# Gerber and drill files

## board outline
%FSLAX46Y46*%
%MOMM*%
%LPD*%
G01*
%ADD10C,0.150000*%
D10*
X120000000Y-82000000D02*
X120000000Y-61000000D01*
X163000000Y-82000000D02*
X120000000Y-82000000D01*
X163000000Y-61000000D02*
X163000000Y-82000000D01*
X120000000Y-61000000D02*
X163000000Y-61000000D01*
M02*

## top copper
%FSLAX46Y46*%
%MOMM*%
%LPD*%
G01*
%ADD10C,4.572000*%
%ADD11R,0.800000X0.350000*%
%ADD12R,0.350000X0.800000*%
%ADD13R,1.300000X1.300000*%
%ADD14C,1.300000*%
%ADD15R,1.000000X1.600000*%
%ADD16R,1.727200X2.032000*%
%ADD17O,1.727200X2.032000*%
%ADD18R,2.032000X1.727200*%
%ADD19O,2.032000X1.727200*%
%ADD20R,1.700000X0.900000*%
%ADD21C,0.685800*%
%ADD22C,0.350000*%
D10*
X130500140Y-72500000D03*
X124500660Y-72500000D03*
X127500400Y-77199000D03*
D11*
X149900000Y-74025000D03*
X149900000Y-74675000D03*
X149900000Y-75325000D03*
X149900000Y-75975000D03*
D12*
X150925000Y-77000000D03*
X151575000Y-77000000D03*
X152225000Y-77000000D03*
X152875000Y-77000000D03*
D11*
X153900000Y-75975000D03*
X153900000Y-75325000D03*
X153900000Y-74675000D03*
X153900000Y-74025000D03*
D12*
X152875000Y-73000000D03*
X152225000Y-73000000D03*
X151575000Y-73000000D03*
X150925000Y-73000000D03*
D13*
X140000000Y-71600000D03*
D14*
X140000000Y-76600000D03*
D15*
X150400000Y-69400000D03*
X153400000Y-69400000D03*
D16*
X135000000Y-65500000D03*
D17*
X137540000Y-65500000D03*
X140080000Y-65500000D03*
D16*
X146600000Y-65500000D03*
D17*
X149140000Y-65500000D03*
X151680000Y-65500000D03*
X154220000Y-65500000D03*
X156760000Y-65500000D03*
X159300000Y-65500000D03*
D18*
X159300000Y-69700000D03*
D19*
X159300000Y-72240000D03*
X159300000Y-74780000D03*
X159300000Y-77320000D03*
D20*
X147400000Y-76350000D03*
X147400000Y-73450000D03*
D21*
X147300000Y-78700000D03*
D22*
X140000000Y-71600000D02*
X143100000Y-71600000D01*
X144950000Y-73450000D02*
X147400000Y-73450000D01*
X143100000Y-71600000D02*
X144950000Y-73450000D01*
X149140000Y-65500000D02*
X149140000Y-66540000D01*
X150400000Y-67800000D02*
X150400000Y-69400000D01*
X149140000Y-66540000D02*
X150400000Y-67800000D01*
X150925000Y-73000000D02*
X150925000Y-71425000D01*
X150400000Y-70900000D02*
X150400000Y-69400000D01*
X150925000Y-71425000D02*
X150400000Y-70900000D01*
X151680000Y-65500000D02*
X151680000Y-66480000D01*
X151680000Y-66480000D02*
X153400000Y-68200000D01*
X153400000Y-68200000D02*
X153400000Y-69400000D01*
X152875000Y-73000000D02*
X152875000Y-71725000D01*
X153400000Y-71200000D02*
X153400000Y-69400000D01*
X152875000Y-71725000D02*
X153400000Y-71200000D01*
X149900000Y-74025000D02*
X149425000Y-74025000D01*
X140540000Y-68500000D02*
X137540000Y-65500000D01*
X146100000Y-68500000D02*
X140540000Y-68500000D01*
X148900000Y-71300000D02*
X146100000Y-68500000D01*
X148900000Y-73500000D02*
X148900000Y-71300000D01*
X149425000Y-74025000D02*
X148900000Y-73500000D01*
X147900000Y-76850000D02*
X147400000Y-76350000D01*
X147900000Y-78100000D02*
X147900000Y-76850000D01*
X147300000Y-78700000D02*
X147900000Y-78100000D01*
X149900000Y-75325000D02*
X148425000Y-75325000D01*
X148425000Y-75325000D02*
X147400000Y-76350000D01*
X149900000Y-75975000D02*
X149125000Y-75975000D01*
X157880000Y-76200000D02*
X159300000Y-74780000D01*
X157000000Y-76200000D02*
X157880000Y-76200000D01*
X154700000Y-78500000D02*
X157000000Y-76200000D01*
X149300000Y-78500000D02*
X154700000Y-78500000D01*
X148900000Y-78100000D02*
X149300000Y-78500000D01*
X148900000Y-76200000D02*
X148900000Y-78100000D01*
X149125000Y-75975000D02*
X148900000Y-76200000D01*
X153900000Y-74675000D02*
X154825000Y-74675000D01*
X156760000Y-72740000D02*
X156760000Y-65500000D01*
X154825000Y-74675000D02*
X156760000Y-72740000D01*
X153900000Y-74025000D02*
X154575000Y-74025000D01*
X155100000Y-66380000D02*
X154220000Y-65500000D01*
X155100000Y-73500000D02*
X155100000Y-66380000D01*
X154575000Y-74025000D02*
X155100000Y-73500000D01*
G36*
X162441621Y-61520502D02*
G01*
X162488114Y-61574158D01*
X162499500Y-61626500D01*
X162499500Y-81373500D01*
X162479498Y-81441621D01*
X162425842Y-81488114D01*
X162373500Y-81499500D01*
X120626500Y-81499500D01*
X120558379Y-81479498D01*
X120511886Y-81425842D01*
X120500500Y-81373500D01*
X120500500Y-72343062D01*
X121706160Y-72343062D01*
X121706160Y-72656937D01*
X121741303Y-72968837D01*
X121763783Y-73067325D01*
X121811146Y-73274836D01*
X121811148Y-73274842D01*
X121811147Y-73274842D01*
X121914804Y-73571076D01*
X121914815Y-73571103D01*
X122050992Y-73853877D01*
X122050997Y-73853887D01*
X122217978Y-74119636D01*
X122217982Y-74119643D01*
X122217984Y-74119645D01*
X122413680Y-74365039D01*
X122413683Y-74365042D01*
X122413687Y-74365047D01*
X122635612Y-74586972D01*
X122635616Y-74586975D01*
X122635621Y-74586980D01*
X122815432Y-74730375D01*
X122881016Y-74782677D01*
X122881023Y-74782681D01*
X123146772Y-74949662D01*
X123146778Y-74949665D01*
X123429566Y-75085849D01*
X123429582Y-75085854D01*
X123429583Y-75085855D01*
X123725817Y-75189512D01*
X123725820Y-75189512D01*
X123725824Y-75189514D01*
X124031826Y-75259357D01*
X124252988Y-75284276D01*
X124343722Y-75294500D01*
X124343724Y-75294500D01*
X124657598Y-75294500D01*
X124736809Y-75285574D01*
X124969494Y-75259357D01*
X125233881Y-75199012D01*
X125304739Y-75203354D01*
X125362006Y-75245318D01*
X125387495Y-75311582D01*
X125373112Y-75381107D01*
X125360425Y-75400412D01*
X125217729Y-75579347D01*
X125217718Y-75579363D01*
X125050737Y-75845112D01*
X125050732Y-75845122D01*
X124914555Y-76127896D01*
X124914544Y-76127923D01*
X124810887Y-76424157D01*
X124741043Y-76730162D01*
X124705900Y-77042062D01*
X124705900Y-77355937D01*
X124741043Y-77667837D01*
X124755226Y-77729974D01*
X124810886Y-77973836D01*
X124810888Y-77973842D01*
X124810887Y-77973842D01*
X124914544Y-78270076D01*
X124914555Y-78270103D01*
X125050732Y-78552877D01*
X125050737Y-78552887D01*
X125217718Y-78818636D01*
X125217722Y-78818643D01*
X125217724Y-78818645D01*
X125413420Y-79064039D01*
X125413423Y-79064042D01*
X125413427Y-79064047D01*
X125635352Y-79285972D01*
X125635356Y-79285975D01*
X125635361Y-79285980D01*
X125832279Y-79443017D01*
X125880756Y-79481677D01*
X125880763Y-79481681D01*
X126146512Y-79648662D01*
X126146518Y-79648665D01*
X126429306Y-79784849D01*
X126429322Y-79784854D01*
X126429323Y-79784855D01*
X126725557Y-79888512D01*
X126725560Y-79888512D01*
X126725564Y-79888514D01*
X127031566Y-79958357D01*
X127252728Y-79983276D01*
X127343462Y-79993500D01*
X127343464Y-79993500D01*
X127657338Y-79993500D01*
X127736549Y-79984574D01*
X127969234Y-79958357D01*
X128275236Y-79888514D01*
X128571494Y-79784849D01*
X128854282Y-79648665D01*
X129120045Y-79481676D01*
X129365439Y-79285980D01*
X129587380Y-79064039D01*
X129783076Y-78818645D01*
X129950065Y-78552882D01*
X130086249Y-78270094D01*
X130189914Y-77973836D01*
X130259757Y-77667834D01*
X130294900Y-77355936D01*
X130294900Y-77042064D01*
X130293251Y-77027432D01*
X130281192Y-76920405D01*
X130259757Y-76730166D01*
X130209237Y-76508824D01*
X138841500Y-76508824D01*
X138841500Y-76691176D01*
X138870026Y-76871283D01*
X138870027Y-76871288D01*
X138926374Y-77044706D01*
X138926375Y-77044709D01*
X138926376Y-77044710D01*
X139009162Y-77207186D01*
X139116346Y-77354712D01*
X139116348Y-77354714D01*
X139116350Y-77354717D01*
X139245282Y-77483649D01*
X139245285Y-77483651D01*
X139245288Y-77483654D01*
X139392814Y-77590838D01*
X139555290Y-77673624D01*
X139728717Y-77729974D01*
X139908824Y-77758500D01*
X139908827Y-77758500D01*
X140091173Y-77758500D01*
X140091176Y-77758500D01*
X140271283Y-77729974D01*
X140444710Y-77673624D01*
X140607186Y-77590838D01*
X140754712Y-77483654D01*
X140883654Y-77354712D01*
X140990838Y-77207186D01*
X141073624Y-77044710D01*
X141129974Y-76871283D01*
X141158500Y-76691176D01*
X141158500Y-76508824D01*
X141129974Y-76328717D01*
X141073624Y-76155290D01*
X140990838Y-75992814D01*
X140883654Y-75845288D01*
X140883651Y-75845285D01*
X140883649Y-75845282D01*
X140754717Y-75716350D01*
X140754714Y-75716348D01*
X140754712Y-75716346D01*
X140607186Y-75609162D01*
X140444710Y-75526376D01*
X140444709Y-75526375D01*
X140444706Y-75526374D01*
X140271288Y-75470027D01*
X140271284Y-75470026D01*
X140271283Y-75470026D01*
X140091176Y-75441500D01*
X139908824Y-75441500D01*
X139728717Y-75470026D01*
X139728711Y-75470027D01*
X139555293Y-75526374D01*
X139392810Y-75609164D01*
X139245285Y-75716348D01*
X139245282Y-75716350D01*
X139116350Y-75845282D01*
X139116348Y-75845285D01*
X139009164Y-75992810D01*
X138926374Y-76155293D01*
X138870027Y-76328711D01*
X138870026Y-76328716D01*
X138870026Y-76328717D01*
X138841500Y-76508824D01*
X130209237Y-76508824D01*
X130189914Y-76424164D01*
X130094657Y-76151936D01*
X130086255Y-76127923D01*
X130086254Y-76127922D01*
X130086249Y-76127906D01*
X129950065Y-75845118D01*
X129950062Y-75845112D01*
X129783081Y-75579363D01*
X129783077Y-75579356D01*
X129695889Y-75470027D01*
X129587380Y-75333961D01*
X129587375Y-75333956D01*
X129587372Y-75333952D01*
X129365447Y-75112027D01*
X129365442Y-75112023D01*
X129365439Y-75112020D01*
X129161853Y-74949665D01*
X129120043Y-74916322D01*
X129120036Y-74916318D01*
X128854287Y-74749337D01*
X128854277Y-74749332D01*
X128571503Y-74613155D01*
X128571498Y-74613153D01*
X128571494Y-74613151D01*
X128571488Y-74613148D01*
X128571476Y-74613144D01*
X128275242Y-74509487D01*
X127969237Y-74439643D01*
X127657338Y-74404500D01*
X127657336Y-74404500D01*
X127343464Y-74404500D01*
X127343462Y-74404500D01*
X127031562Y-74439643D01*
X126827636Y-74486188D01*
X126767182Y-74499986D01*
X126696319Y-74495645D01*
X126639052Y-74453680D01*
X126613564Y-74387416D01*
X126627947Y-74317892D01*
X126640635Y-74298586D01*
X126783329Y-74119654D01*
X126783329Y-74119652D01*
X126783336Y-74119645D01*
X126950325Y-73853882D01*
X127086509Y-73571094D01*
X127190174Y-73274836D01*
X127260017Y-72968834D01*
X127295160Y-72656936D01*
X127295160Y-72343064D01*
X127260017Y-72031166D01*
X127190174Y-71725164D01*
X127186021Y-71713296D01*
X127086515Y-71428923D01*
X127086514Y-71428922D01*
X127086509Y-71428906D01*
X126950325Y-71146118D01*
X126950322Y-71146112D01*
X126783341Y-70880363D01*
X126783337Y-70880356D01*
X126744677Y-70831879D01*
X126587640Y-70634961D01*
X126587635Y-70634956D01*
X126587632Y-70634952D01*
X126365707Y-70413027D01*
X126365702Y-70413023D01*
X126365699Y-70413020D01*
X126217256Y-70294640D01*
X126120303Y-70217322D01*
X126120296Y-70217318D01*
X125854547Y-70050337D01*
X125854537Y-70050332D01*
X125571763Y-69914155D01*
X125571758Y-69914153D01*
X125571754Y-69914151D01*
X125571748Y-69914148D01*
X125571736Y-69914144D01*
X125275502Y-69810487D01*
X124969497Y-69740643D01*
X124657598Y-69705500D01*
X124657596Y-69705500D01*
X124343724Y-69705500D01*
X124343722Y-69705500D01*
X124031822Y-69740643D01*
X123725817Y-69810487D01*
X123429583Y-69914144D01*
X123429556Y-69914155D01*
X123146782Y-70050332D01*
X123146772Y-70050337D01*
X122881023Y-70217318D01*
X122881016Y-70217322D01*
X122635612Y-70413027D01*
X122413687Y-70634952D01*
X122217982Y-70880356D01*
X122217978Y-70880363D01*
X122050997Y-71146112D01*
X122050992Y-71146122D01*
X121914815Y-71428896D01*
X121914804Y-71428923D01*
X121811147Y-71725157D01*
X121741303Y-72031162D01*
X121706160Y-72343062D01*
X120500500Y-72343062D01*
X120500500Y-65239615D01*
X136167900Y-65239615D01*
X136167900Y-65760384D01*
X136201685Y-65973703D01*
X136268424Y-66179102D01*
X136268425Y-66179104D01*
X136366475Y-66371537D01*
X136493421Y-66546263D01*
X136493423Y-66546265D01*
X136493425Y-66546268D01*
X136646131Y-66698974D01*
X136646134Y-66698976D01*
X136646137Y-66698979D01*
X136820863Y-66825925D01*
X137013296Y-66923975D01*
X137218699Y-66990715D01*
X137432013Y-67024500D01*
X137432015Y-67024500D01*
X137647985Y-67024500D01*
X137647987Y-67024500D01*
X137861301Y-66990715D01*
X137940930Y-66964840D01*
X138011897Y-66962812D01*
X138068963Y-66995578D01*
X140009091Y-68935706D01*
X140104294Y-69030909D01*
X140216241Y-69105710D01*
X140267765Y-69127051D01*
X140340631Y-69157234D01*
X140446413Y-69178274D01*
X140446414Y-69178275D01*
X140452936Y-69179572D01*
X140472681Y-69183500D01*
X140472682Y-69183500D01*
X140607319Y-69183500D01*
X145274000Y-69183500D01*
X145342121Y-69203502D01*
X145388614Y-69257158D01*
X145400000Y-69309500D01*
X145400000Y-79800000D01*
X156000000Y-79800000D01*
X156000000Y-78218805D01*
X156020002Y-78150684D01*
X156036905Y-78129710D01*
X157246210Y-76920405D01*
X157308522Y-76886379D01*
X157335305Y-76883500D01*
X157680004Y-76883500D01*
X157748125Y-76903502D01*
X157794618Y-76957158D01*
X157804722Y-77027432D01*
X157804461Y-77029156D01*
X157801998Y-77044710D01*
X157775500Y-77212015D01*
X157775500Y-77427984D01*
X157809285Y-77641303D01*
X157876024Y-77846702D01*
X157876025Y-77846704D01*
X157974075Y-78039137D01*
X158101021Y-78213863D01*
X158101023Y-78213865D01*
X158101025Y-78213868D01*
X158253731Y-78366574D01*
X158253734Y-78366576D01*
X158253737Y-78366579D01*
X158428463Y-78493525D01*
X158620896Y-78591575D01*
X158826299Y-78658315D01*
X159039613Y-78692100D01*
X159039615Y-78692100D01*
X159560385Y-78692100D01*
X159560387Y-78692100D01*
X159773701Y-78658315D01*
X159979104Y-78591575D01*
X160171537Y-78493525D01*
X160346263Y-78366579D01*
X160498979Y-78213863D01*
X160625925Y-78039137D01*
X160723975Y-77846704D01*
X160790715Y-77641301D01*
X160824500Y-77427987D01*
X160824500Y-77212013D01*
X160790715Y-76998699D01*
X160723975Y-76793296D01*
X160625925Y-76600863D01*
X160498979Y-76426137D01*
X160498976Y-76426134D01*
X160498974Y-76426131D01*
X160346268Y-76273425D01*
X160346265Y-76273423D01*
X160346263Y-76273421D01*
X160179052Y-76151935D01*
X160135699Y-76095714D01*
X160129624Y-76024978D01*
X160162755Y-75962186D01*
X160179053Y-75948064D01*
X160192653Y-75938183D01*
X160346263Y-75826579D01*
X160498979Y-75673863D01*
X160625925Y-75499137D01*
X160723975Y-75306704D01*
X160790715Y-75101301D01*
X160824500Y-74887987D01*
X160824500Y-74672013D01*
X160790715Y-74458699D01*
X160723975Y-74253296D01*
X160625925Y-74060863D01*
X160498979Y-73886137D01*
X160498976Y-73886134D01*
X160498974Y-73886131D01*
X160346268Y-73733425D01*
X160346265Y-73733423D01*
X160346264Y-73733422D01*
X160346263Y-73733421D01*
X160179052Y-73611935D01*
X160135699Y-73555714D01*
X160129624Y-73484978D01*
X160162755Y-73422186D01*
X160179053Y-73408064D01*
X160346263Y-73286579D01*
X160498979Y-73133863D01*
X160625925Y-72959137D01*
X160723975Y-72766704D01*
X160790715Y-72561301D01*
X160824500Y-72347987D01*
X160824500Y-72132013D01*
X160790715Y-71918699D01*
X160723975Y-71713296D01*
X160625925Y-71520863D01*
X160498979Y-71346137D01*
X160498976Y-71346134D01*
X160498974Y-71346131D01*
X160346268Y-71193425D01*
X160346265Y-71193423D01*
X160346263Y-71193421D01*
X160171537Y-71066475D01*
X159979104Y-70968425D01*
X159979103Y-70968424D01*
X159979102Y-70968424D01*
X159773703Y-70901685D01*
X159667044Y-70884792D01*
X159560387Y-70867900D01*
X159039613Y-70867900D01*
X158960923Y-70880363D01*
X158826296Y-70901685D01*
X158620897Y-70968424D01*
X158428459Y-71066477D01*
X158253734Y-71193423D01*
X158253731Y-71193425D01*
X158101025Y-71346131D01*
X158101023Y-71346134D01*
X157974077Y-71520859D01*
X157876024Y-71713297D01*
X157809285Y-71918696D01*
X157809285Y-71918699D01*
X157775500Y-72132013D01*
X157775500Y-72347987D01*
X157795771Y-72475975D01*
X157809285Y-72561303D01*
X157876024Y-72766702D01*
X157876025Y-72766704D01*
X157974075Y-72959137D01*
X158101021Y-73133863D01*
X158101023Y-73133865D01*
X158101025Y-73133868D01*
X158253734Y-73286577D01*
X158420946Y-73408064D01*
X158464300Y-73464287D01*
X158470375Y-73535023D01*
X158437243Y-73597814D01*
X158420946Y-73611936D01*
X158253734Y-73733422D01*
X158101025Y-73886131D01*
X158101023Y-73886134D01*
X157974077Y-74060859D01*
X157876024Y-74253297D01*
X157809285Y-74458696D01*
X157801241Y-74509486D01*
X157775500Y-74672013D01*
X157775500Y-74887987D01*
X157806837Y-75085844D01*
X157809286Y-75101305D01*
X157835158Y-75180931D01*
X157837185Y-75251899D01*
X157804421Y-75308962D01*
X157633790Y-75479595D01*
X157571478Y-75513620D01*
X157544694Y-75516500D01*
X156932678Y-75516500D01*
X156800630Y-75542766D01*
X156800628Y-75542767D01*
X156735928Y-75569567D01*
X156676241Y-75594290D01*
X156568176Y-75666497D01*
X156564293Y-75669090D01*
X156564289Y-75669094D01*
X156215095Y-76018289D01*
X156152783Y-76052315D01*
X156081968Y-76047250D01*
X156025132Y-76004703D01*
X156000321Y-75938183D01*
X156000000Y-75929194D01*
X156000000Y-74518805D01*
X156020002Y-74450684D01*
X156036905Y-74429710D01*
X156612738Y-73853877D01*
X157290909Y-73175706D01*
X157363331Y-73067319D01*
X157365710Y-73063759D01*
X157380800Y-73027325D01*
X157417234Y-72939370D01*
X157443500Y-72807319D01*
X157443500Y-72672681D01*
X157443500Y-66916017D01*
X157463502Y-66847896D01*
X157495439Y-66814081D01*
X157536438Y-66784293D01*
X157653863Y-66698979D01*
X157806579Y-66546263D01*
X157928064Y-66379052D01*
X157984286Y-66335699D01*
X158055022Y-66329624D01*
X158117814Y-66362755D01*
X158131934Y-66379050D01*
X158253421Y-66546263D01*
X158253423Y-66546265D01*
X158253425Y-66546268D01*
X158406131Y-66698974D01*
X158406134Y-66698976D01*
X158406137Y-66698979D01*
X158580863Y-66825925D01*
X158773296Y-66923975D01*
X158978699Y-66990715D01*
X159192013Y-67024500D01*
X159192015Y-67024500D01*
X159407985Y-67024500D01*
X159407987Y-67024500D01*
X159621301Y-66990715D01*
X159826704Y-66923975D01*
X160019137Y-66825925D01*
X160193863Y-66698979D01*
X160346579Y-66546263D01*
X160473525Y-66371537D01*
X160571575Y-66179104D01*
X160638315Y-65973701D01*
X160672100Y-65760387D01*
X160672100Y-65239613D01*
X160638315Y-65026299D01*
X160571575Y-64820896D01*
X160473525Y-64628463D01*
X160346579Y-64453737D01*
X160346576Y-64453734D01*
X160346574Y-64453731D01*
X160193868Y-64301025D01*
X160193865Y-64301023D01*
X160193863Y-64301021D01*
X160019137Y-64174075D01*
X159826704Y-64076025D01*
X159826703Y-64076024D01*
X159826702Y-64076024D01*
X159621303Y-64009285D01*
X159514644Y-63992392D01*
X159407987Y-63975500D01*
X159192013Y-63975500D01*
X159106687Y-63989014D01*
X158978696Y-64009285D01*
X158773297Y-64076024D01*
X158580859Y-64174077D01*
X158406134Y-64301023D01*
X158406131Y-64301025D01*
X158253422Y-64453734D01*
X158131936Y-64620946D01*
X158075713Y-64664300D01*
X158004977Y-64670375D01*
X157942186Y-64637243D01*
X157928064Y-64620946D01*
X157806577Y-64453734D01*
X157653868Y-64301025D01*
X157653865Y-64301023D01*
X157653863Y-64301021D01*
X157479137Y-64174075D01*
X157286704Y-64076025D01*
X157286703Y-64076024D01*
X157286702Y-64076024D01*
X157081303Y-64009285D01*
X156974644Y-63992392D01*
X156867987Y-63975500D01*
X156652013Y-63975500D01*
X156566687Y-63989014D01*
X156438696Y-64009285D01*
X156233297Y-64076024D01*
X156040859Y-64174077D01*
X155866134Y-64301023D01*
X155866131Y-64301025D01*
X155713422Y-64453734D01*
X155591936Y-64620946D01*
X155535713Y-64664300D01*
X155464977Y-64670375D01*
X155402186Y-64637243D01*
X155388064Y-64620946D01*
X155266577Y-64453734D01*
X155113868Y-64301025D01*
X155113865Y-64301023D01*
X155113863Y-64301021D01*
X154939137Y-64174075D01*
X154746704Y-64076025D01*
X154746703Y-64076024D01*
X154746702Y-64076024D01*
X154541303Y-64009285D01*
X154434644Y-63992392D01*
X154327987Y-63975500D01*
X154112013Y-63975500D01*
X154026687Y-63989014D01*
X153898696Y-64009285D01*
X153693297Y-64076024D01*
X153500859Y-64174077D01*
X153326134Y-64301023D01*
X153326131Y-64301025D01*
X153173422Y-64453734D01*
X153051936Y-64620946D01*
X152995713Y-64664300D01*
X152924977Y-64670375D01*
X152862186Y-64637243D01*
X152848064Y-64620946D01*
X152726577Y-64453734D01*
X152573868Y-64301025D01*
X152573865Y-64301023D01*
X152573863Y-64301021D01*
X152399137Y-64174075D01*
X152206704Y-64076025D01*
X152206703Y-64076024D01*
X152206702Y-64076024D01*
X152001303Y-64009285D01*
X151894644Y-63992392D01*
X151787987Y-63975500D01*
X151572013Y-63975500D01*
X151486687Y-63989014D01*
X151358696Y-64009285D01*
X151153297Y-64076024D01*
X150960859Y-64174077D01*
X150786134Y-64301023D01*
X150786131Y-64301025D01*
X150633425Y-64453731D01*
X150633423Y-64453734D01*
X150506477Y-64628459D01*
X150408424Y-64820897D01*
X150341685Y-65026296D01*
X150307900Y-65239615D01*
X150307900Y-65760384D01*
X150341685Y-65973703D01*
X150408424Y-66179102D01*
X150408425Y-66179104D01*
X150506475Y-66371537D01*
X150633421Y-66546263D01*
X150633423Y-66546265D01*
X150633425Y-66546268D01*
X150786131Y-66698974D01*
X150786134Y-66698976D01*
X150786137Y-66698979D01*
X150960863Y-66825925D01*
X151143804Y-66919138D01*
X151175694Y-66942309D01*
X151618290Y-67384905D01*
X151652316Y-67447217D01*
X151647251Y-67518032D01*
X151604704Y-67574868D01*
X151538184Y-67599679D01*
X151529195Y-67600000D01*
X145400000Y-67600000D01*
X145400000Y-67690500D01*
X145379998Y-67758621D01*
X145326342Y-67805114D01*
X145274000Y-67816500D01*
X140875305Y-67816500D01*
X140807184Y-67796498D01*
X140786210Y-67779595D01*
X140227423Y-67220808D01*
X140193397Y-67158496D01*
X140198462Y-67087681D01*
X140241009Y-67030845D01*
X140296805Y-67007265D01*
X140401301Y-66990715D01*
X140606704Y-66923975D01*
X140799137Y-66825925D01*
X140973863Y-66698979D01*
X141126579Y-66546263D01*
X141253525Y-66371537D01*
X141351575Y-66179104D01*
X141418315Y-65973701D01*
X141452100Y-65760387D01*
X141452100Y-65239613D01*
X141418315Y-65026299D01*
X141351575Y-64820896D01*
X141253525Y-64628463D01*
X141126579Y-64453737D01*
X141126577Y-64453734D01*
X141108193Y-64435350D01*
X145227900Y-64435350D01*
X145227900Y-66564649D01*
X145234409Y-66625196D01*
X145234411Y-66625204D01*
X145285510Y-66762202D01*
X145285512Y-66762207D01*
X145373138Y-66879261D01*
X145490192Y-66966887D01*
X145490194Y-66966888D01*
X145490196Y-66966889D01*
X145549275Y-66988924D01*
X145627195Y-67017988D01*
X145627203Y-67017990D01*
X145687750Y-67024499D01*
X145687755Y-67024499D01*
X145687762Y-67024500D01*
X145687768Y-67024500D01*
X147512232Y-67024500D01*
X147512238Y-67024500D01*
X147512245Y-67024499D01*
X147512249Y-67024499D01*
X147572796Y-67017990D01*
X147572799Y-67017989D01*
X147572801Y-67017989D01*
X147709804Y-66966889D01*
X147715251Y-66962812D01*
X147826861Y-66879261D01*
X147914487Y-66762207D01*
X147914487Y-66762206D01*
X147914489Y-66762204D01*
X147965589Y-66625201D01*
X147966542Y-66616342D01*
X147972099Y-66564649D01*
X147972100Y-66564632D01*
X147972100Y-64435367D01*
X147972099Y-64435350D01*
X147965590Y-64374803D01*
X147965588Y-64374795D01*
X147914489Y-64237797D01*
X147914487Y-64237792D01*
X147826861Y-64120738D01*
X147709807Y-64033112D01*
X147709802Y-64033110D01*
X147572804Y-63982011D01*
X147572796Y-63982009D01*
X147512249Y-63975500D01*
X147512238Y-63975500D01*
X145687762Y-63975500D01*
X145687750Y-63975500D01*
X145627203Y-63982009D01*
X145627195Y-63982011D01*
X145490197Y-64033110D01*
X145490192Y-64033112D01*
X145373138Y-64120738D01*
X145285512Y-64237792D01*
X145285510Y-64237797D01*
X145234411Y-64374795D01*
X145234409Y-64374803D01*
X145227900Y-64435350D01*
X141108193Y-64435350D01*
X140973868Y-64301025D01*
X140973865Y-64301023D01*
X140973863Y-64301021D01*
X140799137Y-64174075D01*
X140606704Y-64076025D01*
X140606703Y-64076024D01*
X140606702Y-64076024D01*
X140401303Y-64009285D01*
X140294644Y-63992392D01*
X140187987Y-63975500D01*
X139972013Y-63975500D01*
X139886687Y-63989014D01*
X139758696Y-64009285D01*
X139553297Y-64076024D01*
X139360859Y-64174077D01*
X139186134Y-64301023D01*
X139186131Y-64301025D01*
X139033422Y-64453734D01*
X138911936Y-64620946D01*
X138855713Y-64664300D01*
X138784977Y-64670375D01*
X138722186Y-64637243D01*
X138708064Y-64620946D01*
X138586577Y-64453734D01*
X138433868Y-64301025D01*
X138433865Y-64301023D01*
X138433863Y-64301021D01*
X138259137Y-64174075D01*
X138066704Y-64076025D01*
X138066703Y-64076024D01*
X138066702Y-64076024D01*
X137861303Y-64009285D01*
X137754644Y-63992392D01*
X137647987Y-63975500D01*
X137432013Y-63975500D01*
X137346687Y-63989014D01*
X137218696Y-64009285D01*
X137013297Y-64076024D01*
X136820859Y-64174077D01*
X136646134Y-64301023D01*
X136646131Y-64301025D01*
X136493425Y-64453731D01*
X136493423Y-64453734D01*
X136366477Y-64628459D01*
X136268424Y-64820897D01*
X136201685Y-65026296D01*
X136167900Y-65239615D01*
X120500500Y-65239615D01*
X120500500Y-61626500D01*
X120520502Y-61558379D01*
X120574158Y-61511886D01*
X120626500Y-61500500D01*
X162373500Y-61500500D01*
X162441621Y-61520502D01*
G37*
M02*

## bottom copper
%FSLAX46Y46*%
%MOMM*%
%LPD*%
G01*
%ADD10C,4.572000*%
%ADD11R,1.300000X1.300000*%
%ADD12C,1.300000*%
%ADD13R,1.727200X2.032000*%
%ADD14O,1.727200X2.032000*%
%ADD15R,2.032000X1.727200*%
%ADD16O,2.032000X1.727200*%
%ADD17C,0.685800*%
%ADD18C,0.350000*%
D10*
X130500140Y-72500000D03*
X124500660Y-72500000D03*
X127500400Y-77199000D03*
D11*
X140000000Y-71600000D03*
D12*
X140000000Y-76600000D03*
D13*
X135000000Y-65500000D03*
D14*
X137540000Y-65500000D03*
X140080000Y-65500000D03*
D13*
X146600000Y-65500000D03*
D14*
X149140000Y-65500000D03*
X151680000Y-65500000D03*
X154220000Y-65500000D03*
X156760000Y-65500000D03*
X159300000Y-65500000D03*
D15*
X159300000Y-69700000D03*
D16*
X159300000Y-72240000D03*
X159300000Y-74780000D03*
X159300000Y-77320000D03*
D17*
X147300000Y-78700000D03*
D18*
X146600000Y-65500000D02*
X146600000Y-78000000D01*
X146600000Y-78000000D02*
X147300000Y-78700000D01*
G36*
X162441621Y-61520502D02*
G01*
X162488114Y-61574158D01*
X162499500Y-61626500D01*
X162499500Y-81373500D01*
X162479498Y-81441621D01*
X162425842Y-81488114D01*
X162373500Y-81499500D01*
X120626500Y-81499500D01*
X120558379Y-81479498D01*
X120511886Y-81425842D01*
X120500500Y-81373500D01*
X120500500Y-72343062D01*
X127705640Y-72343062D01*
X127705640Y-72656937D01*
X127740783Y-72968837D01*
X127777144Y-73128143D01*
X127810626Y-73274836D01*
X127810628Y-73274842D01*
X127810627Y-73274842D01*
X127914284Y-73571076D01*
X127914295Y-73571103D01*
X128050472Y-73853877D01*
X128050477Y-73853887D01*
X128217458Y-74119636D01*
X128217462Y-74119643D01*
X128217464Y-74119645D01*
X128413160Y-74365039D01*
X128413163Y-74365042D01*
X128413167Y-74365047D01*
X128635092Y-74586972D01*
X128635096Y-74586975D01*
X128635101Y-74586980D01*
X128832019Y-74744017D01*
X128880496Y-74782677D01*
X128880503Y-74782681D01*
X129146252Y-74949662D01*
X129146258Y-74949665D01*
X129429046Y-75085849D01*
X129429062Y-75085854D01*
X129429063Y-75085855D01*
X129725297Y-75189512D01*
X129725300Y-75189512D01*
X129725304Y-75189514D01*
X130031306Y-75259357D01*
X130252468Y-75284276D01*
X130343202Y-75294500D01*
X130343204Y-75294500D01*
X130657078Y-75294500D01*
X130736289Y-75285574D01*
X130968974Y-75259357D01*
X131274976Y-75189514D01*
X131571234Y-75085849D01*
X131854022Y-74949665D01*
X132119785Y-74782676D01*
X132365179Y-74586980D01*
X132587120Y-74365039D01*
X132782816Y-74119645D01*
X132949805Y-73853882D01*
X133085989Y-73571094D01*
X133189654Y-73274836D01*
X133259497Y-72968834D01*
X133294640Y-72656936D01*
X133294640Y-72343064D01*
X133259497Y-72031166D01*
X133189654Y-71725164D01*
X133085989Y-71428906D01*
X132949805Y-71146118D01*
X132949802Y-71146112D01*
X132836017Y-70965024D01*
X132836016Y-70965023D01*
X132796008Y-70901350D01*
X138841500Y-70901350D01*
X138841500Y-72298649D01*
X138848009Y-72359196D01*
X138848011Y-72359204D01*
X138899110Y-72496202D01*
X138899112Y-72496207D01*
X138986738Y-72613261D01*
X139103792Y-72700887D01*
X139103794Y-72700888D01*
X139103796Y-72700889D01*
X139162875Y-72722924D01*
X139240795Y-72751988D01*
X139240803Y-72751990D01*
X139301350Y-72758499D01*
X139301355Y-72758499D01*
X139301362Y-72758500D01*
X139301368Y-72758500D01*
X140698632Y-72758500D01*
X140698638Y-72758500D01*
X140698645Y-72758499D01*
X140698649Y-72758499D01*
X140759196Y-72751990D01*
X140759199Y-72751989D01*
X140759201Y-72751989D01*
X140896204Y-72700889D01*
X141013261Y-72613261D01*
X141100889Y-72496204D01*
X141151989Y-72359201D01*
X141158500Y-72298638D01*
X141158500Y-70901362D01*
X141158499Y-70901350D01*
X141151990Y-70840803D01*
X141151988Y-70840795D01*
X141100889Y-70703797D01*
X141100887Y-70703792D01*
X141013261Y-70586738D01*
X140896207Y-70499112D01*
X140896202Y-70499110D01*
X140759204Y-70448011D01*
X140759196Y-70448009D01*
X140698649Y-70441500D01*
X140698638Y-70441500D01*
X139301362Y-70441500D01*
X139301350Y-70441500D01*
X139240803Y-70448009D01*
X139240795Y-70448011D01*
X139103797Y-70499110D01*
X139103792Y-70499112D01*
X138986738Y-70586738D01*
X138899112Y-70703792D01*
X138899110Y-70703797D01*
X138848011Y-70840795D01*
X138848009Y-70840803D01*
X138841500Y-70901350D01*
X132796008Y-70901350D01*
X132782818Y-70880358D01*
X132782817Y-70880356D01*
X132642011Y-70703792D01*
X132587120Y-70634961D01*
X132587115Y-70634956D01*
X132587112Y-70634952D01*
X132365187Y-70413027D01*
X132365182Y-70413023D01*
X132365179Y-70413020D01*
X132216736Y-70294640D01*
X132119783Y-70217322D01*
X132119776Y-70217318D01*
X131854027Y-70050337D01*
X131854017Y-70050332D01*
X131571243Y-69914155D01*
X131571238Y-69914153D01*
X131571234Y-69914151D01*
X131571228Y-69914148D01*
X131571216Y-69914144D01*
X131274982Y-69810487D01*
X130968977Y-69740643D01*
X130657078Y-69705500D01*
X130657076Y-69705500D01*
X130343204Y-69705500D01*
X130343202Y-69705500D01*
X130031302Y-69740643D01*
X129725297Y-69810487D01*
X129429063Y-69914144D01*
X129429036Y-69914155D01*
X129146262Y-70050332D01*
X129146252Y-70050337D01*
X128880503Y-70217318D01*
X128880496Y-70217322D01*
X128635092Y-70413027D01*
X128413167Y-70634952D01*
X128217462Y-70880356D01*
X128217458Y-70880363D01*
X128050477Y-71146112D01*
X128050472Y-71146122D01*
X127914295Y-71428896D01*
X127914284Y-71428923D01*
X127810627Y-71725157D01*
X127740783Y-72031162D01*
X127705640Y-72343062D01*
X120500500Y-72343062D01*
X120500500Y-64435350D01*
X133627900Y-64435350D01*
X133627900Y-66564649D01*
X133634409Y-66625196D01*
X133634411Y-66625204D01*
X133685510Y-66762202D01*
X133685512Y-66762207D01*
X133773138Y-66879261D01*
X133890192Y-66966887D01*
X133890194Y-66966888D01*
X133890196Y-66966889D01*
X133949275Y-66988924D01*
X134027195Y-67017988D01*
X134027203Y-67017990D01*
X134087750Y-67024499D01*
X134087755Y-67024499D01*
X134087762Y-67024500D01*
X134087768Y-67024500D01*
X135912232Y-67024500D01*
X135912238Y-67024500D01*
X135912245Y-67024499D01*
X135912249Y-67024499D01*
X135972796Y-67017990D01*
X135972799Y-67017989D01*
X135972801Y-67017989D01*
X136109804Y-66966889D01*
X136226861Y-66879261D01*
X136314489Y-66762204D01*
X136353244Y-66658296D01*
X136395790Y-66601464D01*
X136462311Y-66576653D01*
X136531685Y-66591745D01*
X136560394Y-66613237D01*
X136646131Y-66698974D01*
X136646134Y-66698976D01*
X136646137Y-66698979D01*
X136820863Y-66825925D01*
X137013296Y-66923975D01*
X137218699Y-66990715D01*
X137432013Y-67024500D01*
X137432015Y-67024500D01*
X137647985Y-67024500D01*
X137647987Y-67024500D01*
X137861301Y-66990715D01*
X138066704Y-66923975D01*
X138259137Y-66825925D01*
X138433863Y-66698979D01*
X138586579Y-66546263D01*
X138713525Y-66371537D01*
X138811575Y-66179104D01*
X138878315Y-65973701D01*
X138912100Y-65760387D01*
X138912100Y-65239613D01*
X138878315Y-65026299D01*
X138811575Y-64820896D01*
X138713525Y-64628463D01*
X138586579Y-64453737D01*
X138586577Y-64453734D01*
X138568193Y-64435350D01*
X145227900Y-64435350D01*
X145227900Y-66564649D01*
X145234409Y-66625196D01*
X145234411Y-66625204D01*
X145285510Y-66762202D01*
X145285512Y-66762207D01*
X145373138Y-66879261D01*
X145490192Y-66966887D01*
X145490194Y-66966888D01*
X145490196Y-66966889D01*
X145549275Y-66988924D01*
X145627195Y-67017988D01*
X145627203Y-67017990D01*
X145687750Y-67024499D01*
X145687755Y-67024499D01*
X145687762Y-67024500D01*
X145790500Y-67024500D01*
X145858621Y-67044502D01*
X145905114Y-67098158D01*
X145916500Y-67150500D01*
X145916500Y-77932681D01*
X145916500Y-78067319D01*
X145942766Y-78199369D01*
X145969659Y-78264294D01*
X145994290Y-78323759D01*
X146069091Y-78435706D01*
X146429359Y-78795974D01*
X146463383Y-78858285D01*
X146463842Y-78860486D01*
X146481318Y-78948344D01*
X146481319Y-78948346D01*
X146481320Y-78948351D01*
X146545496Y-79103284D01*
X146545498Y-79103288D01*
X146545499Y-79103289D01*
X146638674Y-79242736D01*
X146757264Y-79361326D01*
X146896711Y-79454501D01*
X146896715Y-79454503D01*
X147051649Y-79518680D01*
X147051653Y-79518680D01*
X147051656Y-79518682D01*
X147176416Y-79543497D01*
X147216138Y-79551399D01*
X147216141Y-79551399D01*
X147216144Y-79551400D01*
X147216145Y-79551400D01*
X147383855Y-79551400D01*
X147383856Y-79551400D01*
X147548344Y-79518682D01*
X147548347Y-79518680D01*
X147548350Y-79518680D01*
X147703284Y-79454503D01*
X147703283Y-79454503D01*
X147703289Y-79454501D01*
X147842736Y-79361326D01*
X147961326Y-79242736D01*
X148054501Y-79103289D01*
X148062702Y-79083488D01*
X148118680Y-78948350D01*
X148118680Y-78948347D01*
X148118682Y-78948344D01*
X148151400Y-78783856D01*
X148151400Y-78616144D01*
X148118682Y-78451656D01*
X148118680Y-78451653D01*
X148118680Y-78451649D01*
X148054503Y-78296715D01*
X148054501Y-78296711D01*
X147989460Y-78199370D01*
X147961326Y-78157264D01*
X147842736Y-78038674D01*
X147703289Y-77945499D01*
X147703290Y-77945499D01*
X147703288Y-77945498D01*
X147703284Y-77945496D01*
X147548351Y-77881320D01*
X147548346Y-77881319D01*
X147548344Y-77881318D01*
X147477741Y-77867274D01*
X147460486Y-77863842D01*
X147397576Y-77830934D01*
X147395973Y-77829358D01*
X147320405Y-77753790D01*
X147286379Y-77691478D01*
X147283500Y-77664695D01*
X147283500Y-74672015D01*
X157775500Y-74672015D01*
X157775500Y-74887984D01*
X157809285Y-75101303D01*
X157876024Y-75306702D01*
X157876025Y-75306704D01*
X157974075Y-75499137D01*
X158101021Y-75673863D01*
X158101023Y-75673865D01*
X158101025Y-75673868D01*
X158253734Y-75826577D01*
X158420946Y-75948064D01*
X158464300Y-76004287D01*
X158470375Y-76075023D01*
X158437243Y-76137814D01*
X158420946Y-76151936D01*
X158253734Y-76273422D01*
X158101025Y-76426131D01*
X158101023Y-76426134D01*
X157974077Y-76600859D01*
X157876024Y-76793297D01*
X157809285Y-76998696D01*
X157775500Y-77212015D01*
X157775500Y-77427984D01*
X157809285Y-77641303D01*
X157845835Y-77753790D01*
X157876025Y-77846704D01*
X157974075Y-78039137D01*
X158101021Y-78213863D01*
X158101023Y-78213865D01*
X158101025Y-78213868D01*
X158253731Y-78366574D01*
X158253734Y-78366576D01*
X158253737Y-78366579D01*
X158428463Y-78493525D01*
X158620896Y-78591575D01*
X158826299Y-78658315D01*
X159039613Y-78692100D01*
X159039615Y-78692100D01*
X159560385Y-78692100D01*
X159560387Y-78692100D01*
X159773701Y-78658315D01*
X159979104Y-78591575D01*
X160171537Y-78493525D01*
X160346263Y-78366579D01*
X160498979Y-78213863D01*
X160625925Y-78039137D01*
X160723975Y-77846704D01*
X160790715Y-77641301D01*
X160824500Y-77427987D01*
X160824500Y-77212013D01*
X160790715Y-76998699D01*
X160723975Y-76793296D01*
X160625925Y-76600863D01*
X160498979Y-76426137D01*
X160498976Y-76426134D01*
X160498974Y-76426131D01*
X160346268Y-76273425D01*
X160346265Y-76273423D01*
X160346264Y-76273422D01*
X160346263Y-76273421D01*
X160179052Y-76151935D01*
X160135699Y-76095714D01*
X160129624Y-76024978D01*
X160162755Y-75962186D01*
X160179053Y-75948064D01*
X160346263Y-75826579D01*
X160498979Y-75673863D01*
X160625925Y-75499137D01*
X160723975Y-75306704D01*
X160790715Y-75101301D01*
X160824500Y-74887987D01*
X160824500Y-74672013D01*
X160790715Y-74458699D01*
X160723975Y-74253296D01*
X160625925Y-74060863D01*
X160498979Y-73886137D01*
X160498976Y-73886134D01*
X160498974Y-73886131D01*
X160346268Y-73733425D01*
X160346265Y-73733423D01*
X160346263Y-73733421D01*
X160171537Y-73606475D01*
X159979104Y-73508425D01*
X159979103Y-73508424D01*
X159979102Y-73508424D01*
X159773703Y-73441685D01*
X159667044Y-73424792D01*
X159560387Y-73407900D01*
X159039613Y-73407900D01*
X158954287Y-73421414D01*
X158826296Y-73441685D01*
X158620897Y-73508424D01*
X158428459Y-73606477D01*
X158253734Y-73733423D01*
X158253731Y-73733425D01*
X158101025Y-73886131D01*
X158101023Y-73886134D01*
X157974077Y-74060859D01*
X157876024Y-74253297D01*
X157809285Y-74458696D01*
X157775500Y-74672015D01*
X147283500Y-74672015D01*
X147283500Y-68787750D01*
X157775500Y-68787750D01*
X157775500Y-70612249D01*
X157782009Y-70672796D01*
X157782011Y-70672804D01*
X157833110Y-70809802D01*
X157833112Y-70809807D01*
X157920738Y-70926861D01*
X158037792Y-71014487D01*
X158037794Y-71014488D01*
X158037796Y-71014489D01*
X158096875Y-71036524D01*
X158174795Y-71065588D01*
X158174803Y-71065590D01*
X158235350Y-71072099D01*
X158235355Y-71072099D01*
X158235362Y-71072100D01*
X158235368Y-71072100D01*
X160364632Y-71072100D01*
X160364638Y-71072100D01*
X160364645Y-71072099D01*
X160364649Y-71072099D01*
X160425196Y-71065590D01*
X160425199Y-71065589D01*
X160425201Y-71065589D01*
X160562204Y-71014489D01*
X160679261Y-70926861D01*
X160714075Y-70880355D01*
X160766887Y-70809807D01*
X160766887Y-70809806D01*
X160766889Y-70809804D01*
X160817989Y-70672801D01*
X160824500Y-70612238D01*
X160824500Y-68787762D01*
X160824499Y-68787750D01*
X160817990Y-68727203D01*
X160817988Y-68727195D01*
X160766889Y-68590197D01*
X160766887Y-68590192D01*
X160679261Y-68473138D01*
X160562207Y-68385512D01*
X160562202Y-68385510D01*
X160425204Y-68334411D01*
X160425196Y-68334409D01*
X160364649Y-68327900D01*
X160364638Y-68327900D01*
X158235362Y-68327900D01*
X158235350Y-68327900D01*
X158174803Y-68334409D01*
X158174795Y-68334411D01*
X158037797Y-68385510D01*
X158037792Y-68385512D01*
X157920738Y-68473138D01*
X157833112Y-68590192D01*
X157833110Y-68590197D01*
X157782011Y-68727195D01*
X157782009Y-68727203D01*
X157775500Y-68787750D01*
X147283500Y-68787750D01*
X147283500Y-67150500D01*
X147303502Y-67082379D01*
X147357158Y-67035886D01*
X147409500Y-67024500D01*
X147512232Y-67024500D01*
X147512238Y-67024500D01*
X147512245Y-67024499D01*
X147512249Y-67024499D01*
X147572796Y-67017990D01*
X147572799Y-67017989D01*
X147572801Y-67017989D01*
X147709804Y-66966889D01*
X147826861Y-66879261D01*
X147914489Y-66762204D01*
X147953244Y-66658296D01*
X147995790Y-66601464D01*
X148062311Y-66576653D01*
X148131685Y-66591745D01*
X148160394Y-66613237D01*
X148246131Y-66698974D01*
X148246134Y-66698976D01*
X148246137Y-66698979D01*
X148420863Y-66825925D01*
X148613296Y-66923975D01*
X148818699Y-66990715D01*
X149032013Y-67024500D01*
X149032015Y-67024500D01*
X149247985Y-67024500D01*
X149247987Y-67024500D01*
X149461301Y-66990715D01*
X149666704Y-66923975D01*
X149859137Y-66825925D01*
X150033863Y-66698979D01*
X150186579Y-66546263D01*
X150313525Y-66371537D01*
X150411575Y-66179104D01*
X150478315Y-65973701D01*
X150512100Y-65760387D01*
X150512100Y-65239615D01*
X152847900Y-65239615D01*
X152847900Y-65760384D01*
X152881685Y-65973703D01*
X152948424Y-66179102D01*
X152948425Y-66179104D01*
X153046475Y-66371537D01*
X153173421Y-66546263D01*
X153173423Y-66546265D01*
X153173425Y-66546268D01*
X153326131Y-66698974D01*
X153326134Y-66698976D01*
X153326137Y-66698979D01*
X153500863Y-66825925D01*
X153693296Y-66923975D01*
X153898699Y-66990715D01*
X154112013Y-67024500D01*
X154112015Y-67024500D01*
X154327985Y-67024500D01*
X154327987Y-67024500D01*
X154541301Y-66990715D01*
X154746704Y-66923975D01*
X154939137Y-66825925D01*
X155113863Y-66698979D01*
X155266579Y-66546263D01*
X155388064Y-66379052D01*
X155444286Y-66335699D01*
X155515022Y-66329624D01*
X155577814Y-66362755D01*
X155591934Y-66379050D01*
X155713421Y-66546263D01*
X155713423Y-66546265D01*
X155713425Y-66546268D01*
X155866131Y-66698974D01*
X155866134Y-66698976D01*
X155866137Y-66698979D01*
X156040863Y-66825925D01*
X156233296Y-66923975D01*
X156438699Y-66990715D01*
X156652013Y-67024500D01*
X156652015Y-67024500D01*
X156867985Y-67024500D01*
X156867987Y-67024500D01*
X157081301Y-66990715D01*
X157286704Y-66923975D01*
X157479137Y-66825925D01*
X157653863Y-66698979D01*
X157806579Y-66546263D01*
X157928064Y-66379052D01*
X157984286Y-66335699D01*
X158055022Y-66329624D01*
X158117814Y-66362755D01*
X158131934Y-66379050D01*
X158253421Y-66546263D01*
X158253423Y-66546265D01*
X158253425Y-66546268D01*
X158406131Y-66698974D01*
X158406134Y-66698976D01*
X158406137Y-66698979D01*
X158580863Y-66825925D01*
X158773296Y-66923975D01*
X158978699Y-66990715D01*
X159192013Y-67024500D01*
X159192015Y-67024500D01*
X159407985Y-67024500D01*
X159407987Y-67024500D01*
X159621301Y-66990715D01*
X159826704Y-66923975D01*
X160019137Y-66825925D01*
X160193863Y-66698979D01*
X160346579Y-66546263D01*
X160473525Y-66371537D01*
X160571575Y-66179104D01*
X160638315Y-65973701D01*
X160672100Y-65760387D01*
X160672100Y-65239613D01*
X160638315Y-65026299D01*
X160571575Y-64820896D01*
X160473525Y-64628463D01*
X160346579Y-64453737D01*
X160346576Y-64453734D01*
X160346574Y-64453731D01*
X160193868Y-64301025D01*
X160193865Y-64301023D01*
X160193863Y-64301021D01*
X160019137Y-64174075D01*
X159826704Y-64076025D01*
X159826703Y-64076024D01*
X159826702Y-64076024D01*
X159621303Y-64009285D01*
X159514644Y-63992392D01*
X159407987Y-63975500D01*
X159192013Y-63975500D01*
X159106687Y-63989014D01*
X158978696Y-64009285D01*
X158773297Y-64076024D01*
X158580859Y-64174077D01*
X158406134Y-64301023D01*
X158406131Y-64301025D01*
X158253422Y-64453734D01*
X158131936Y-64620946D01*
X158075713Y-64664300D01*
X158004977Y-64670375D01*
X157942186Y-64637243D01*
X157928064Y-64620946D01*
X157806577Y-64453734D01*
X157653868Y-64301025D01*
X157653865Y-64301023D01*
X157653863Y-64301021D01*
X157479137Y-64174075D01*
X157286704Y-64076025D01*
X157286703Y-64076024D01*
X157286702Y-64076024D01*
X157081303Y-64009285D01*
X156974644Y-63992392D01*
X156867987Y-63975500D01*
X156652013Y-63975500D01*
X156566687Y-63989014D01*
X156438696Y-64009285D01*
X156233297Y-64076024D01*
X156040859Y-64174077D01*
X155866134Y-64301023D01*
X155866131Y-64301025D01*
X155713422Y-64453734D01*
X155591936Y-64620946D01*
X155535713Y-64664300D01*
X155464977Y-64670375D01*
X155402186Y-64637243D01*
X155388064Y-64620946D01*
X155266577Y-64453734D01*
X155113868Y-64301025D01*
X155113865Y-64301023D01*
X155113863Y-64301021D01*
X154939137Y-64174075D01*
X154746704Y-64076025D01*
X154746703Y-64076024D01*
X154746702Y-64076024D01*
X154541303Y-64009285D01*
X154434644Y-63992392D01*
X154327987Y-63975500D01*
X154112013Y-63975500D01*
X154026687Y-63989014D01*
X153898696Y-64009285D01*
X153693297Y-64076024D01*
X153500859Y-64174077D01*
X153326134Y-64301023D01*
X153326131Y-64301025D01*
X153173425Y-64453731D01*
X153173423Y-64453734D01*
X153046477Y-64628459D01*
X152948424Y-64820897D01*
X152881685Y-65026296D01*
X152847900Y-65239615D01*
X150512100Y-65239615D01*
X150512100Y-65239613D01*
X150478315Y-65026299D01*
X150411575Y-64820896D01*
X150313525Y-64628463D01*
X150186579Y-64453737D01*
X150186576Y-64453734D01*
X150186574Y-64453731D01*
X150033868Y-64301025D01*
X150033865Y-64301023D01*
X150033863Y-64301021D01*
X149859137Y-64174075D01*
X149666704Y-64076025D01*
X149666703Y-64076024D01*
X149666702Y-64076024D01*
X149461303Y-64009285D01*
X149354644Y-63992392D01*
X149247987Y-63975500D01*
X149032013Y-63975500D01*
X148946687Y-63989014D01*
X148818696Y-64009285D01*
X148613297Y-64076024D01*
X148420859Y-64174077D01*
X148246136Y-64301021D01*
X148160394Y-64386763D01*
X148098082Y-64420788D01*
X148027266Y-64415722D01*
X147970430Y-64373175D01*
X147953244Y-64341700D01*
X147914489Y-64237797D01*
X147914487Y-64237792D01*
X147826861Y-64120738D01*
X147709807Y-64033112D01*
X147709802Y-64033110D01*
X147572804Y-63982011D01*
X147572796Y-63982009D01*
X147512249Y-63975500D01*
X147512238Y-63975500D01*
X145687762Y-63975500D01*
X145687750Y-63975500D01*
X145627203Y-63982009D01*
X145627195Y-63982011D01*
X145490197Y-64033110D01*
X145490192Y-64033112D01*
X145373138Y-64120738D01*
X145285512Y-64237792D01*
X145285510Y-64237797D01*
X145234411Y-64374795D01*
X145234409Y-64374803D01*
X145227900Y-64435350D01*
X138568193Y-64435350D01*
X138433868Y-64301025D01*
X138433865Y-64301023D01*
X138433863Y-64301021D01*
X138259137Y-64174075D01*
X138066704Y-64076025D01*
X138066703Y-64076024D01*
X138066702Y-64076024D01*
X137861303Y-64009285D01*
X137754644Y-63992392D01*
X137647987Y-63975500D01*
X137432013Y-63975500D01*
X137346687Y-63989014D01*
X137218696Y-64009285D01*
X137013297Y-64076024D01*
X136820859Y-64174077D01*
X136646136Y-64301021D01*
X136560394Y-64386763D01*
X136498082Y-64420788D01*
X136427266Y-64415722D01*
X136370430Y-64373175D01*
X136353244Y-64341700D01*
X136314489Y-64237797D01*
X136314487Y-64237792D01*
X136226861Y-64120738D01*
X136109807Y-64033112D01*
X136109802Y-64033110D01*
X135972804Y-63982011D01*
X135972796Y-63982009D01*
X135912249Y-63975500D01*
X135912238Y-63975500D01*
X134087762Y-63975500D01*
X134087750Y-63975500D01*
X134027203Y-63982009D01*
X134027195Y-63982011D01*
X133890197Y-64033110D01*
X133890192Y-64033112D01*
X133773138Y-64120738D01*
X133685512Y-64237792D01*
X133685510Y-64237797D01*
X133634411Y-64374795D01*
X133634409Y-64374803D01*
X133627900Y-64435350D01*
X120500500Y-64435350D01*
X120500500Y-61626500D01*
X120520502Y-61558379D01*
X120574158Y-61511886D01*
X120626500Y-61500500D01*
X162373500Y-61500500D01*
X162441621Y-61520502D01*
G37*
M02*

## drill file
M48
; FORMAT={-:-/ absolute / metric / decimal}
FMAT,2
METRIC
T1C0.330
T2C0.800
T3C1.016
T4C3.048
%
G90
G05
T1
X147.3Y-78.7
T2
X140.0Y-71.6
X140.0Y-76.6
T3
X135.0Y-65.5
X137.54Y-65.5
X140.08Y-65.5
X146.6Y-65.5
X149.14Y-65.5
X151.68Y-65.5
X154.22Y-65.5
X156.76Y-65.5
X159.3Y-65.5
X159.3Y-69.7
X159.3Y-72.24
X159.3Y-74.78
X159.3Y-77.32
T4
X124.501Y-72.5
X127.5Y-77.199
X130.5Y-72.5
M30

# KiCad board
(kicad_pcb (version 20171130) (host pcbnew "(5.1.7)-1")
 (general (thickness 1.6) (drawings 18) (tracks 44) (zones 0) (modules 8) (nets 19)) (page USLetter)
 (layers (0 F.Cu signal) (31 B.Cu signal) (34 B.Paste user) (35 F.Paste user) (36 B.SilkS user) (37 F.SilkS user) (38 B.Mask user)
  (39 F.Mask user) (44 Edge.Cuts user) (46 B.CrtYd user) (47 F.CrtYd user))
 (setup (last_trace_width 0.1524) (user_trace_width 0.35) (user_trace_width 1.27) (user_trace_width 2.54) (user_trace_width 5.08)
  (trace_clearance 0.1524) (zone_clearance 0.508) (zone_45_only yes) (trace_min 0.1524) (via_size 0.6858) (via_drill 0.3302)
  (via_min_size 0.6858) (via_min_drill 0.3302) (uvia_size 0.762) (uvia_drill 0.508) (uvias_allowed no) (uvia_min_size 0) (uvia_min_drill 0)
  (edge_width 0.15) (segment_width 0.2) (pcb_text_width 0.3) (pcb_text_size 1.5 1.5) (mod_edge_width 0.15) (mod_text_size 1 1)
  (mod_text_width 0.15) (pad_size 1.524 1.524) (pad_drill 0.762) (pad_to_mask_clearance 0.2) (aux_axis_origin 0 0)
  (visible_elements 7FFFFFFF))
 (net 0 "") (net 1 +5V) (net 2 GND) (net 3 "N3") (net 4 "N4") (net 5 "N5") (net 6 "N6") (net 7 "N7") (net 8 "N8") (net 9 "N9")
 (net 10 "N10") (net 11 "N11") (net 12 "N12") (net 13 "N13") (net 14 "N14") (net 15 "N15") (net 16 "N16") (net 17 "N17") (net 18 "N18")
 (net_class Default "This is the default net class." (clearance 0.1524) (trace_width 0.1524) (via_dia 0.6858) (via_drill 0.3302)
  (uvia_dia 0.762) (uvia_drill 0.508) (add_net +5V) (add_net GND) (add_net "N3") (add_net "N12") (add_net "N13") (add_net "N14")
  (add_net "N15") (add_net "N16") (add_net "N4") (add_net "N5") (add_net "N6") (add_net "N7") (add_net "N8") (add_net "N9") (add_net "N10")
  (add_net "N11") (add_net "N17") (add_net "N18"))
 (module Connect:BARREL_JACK (layer F.Cu) (at 124.3 72.5)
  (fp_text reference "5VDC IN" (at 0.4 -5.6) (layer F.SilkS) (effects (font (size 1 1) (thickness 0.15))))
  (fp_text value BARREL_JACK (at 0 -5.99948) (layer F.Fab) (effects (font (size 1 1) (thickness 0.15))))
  (pad 1 thru_hole circle (at 6.20014 0) (size 4.572 4.572) (drill 3.048) (layers *.Cu *.Mask F.SilkS) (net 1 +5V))
  (pad 2 thru_hole circle (at 0.20066 0) (size 4.572 4.572) (drill oval 3.048) (layers *.Cu *.Mask F.SilkS) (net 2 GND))
  (pad 3 thru_hole circle (at 3.2004 4.699) (size 4.572 4.572) (drill 3.048) (layers *.Cu *.Mask F.SilkS) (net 2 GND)))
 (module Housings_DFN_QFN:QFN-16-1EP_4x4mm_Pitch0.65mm (layer F.Cu) (at 151.9 75)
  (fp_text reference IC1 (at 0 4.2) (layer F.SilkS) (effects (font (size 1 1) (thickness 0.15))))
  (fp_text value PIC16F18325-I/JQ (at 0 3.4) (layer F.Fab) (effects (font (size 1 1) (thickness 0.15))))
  (pad 1 smd rect (at -2 -0.975) (size 0.8 0.35) (layers F.Cu F.Paste F.Mask) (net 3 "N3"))
  (pad 2 smd rect (at -2 -0.325) (size 0.8 0.35) (layers F.Cu F.Paste F.Mask) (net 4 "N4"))
  (pad 3 smd rect (at -2 0.325) (size 0.8 0.35) (layers F.Cu F.Paste F.Mask) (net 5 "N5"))
  (pad 4 smd rect (at -2 0.975) (size 0.8 0.35) (layers F.Cu F.Paste F.Mask) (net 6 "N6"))
  (pad 5 smd rect (at -0.975 2 90) (size 0.8 0.35) (layers F.Cu F.Paste F.Mask) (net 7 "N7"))
  (pad 6 smd rect (at -0.325 2 90) (size 0.8 0.35) (layers F.Cu F.Paste F.Mask) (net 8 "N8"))
  (pad 7 smd rect (at 0.325 2 90) (size 0.8 0.35) (layers F.Cu F.Paste F.Mask) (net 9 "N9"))
  (pad 8 smd rect (at 0.975 2 90) (size 0.8 0.35) (layers F.Cu F.Paste F.Mask) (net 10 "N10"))
  (pad 9 smd rect (at 2 0.975) (size 0.8 0.35) (layers F.Cu F.Paste F.Mask) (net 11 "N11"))
  (pad 10 smd rect (at 2 0.325) (size 0.8 0.35) (layers F.Cu F.Paste F.Mask) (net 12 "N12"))
  (pad 11 smd rect (at 2 -0.325) (size 0.8 0.35) (layers F.Cu F.Paste F.Mask) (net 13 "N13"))
  (pad 12 smd rect (at 2 -0.975) (size 0.8 0.35) (layers F.Cu F.Paste F.Mask) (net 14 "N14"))
  (pad 13 smd rect (at 0.975 -2 90) (size 0.8 0.35) (layers F.Cu F.Paste F.Mask) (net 2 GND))
  (pad 14 smd rect (at 0.325 -2 90) (size 0.8 0.35) (layers F.Cu F.Paste F.Mask) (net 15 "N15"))
  (pad 15 smd rect (at -0.325 -2 90) (size 0.8 0.35) (layers F.Cu F.Paste F.Mask) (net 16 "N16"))
  (pad 16 smd rect (at -0.975 -2 90) (size 0.8 0.35) (layers F.Cu F.Paste F.Mask) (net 1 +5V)))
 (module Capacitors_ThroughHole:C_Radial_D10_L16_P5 (layer F.Cu) (at 140 71.6 270)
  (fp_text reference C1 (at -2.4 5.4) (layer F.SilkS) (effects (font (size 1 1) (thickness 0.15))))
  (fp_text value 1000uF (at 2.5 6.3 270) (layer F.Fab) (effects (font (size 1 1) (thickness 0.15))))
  (pad 1 thru_hole rect (at 0 0 270) (size 1.3 1.3) (drill 0.8) (layers *.Cu *.Mask F.SilkS) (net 1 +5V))
  (pad 2 thru_hole circle (at 5 0 270) (size 1.3 1.3) (drill 0.8) (layers *.Cu *.Mask F.SilkS) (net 2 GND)))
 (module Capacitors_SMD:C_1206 (layer F.Cu) (at 151.9 69.4)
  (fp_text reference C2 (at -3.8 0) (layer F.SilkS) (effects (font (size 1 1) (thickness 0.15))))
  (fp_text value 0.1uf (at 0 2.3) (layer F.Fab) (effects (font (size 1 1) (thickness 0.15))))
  (pad 1 smd rect (at -1.5 0) (size 1 1.6) (layers F.Cu F.Paste F.Mask) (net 1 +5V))
  (pad 2 smd rect (at 1.5 0) (size 1 1.6) (layers F.Cu F.Paste F.Mask) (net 2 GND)))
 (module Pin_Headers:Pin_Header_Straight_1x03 (layer F.Cu) (at 135 65.5 90)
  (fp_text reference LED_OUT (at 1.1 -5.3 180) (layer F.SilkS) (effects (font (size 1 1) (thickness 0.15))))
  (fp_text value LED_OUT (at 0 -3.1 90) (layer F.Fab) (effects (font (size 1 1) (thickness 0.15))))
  (pad 1 thru_hole rect (at 0 0 90) (size 2.032 1.7272) (drill 1.016) (layers *.Cu *.Mask F.SilkS) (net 1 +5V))
  (pad 2 thru_hole oval (at 0 2.54 90) (size 2.032 1.7272) (drill 1.016) (layers *.Cu *.Mask F.SilkS) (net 3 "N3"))
  (pad 3 thru_hole oval (at 0 5.08 90) (size 2.032 1.7272) (drill 1.016) (layers *.Cu *.Mask F.SilkS) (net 2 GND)))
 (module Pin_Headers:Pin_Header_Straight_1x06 (layer F.Cu) (at 146.6 65.5 90)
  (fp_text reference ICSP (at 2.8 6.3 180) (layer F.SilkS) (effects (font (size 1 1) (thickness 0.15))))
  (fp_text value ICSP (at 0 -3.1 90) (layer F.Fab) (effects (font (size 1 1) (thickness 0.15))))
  (pad 1 thru_hole rect (at 0 0 90) (size 2.032 1.7272) (drill 1.016) (layers *.Cu *.Mask F.SilkS) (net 5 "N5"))
  (pad 2 thru_hole oval (at 0 2.54 90) (size 2.032 1.7272) (drill 1.016) (layers *.Cu *.Mask F.SilkS) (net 1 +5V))
  (pad 3 thru_hole oval (at 0 5.08 90) (size 2.032 1.7272) (drill 1.016) (layers *.Cu *.Mask F.SilkS) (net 2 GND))
  (pad 4 thru_hole oval (at 0 7.62 90) (size 2.032 1.7272) (drill 1.016) (layers *.Cu *.Mask F.SilkS) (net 14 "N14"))
  (pad 5 thru_hole oval (at 0 10.16 90) (size 2.032 1.7272) (drill 1.016) (layers *.Cu *.Mask F.SilkS) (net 13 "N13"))
  (pad 6 thru_hole oval (at 0 12.7 90) (size 2.032 1.7272) (drill 1.016) (layers *.Cu *.Mask F.SilkS) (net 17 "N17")))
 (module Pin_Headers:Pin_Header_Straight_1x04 (layer F.Cu) (at 159.3 69.7)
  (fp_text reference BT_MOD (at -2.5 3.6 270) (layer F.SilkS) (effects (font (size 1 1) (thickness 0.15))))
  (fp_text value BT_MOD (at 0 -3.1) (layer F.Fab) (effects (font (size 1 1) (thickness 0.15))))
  (pad 1 thru_hole rect (at 0 0) (size 2.032 1.7272) (drill 1.016) (layers *.Cu *.Mask F.SilkS) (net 1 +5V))
  (pad 2 thru_hole oval (at 0 2.54) (size 2.032 1.7272) (drill 1.016) (layers *.Cu *.Mask F.SilkS) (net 2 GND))
  (pad 3 thru_hole oval (at 0 5.08) (size 2.032 1.7272) (drill 1.016) (layers *.Cu *.Mask F.SilkS) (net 6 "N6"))
  (pad 4 thru_hole oval (at 0 7.62) (size 2.032 1.7272) (drill 1.016) (layers *.Cu *.Mask F.SilkS) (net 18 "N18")))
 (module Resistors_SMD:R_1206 (layer F.Cu) (at 147.4 74.9 90)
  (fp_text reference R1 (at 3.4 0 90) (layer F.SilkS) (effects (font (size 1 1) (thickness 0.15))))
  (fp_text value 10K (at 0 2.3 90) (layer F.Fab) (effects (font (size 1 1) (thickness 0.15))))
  (pad 1 smd rect (at -1.45 0 90) (size 0.9 1.7) (layers F.Cu F.Paste F.Mask) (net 5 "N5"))
  (pad 2 smd rect (at 1.45 0 90) (size 0.9 1.7) (layers F.Cu F.Paste F.Mask) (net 1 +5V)))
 (gr_line (start 120 82) (end 120 61) (angle 90) (layer Edge.Cuts) (width 0.15))
 (gr_line (start 163 82) (end 120 82) (angle 90) (layer Edge.Cuts) (width 0.15))
 (gr_line (start 163 61) (end 163 82) (angle 90) (layer Edge.Cuts) (width 0.15))
 (gr_line (start 120 61) (end 163 61) (angle 90) (layer Edge.Cuts) (width 0.15))
 (segment (start 140 71.6) (end 143.1 71.6) (width 0.35) (layer F.Cu) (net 1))
 (segment (start 144.95 73.45) (end 147.4 73.45) (width 0.35) (layer F.Cu) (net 1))
 (segment (start 143.1 71.6) (end 144.95 73.45) (width 0.35) (layer F.Cu) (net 1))
 (segment (start 149.14 65.5) (end 149.14 66.54) (width 0.35) (layer F.Cu) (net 1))
 (segment (start 150.4 67.8) (end 150.4 69.4) (width 0.35) (layer F.Cu) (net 1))
 (segment (start 149.14 66.54) (end 150.4 67.8) (width 0.35) (layer F.Cu) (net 1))
 (segment (start 150.925 73) (end 150.925 71.425) (width 0.35) (layer F.Cu) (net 1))
 (segment (start 150.4 70.9) (end 150.4 69.4) (width 0.35) (layer F.Cu) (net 1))
 (segment (start 150.925 71.425) (end 150.4 70.9) (width 0.35) (layer F.Cu) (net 1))
 (segment (start 151.68 65.5) (end 151.68 66.48) (width 0.35) (layer F.Cu) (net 2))
 (segment (start 151.68 66.48) (end 153.4 68.2) (width 0.35) (layer F.Cu) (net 2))
 (segment (start 153.4 68.2) (end 153.4 69.4) (width 0.35) (layer F.Cu) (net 2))
 (segment (start 152.875 73) (end 152.875 71.725) (width 0.35) (layer F.Cu) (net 2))
 (segment (start 153.4 71.2) (end 153.4 69.4) (width 0.35) (layer F.Cu) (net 2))
 (segment (start 152.875 71.725) (end 153.4 71.2) (width 0.35) (layer F.Cu) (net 2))
 (segment (start 149.9 74.025) (end 149.425 74.025) (width 0.35) (layer F.Cu) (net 3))
 (segment (start 140.54 68.5) (end 137.54 65.5) (width 0.35) (layer F.Cu) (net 3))
 (segment (start 146.1 68.5) (end 140.54 68.5) (width 0.35) (layer F.Cu) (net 3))
 (segment (start 148.9 71.3) (end 146.1 68.5) (width 0.35) (layer F.Cu) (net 3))
 (segment (start 148.9 73.5) (end 148.9 71.3) (width 0.35) (layer F.Cu) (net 3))
 (segment (start 149.425 74.025) (end 148.9 73.5) (width 0.35) (layer F.Cu) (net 3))
 (segment (start 146.6 65.5) (end 146.6 78) (width 0.35) (layer B.Cu) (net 5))
 (segment (start 147.9 76.85) (end 147.4 76.35) (width 0.35) (layer F.Cu) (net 5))
 (segment (start 147.9 78.1) (end 147.9 76.85) (width 0.35) (layer F.Cu) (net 5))
 (segment (start 147.3 78.7) (end 147.9 78.1) (width 0.35) (layer F.Cu) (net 5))
 (via (at 147.3 78.7) (size 0.6858) (drill 0.3302) (layers F.Cu B.Cu) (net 5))
 (segment (start 146.6 78) (end 147.3 78.7) (width 0.35) (layer B.Cu) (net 5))
 (segment (start 149.9 75.325) (end 148.425 75.325) (width 0.35) (layer F.Cu) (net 5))
 (segment (start 148.425 75.325) (end 147.4 76.35) (width 0.35) (layer F.Cu) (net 5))
 (segment (start 149.9 75.975) (end 149.125 75.975) (width 0.35) (layer F.Cu) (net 6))
 (segment (start 157.88 76.2) (end 159.3 74.78) (width 0.35) (layer F.Cu) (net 6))
 (segment (start 157 76.2) (end 157.88 76.2) (width 0.35) (layer F.Cu) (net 6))
 (segment (start 154.7 78.5) (end 157 76.2) (width 0.35) (layer F.Cu) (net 6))
 (segment (start 149.3 78.5) (end 154.7 78.5) (width 0.35) (layer F.Cu) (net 6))
 (segment (start 148.9 78.1) (end 149.3 78.5) (width 0.35) (layer F.Cu) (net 6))
 (segment (start 148.9 76.2) (end 148.9 78.1) (width 0.35) (layer F.Cu) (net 6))
 (segment (start 149.125 75.975) (end 148.9 76.2) (width 0.35) (layer F.Cu) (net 6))
 (segment (start 153.9 74.675) (end 154.825 74.675) (width 0.35) (layer F.Cu) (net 13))
 (segment (start 156.76 72.74) (end 156.76 65.5) (width 0.35) (layer F.Cu) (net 13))
 (segment (start 154.825 74.675) (end 156.76 72.74) (width 0.35) (layer F.Cu) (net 13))
 (segment (start 153.9 74.025) (end 154.575 74.025) (width 0.35) (layer F.Cu) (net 14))
 (segment (start 155.1 66.38) (end 154.22 65.5) (width 0.35) (layer F.Cu) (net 14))
 (segment (start 155.1 73.5) (end 155.1 66.38) (width 0.35) (layer F.Cu) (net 14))
 (segment (start 154.575 74.025) (end 155.1 73.5) (width 0.35) (layer F.Cu) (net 14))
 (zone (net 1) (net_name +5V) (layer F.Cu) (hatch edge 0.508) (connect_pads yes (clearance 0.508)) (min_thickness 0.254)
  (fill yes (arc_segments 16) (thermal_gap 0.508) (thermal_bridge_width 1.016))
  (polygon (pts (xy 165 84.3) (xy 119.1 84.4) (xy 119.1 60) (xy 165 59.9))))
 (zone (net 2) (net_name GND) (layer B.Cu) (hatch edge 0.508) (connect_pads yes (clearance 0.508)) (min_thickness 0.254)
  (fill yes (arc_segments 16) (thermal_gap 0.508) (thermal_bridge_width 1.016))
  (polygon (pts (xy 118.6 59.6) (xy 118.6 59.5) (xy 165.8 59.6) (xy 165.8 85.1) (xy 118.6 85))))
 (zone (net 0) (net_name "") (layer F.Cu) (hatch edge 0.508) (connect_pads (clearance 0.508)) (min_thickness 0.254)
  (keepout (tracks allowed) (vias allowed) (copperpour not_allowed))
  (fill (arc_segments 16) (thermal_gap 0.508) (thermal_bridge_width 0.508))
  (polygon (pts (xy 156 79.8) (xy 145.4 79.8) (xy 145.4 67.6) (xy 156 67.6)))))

